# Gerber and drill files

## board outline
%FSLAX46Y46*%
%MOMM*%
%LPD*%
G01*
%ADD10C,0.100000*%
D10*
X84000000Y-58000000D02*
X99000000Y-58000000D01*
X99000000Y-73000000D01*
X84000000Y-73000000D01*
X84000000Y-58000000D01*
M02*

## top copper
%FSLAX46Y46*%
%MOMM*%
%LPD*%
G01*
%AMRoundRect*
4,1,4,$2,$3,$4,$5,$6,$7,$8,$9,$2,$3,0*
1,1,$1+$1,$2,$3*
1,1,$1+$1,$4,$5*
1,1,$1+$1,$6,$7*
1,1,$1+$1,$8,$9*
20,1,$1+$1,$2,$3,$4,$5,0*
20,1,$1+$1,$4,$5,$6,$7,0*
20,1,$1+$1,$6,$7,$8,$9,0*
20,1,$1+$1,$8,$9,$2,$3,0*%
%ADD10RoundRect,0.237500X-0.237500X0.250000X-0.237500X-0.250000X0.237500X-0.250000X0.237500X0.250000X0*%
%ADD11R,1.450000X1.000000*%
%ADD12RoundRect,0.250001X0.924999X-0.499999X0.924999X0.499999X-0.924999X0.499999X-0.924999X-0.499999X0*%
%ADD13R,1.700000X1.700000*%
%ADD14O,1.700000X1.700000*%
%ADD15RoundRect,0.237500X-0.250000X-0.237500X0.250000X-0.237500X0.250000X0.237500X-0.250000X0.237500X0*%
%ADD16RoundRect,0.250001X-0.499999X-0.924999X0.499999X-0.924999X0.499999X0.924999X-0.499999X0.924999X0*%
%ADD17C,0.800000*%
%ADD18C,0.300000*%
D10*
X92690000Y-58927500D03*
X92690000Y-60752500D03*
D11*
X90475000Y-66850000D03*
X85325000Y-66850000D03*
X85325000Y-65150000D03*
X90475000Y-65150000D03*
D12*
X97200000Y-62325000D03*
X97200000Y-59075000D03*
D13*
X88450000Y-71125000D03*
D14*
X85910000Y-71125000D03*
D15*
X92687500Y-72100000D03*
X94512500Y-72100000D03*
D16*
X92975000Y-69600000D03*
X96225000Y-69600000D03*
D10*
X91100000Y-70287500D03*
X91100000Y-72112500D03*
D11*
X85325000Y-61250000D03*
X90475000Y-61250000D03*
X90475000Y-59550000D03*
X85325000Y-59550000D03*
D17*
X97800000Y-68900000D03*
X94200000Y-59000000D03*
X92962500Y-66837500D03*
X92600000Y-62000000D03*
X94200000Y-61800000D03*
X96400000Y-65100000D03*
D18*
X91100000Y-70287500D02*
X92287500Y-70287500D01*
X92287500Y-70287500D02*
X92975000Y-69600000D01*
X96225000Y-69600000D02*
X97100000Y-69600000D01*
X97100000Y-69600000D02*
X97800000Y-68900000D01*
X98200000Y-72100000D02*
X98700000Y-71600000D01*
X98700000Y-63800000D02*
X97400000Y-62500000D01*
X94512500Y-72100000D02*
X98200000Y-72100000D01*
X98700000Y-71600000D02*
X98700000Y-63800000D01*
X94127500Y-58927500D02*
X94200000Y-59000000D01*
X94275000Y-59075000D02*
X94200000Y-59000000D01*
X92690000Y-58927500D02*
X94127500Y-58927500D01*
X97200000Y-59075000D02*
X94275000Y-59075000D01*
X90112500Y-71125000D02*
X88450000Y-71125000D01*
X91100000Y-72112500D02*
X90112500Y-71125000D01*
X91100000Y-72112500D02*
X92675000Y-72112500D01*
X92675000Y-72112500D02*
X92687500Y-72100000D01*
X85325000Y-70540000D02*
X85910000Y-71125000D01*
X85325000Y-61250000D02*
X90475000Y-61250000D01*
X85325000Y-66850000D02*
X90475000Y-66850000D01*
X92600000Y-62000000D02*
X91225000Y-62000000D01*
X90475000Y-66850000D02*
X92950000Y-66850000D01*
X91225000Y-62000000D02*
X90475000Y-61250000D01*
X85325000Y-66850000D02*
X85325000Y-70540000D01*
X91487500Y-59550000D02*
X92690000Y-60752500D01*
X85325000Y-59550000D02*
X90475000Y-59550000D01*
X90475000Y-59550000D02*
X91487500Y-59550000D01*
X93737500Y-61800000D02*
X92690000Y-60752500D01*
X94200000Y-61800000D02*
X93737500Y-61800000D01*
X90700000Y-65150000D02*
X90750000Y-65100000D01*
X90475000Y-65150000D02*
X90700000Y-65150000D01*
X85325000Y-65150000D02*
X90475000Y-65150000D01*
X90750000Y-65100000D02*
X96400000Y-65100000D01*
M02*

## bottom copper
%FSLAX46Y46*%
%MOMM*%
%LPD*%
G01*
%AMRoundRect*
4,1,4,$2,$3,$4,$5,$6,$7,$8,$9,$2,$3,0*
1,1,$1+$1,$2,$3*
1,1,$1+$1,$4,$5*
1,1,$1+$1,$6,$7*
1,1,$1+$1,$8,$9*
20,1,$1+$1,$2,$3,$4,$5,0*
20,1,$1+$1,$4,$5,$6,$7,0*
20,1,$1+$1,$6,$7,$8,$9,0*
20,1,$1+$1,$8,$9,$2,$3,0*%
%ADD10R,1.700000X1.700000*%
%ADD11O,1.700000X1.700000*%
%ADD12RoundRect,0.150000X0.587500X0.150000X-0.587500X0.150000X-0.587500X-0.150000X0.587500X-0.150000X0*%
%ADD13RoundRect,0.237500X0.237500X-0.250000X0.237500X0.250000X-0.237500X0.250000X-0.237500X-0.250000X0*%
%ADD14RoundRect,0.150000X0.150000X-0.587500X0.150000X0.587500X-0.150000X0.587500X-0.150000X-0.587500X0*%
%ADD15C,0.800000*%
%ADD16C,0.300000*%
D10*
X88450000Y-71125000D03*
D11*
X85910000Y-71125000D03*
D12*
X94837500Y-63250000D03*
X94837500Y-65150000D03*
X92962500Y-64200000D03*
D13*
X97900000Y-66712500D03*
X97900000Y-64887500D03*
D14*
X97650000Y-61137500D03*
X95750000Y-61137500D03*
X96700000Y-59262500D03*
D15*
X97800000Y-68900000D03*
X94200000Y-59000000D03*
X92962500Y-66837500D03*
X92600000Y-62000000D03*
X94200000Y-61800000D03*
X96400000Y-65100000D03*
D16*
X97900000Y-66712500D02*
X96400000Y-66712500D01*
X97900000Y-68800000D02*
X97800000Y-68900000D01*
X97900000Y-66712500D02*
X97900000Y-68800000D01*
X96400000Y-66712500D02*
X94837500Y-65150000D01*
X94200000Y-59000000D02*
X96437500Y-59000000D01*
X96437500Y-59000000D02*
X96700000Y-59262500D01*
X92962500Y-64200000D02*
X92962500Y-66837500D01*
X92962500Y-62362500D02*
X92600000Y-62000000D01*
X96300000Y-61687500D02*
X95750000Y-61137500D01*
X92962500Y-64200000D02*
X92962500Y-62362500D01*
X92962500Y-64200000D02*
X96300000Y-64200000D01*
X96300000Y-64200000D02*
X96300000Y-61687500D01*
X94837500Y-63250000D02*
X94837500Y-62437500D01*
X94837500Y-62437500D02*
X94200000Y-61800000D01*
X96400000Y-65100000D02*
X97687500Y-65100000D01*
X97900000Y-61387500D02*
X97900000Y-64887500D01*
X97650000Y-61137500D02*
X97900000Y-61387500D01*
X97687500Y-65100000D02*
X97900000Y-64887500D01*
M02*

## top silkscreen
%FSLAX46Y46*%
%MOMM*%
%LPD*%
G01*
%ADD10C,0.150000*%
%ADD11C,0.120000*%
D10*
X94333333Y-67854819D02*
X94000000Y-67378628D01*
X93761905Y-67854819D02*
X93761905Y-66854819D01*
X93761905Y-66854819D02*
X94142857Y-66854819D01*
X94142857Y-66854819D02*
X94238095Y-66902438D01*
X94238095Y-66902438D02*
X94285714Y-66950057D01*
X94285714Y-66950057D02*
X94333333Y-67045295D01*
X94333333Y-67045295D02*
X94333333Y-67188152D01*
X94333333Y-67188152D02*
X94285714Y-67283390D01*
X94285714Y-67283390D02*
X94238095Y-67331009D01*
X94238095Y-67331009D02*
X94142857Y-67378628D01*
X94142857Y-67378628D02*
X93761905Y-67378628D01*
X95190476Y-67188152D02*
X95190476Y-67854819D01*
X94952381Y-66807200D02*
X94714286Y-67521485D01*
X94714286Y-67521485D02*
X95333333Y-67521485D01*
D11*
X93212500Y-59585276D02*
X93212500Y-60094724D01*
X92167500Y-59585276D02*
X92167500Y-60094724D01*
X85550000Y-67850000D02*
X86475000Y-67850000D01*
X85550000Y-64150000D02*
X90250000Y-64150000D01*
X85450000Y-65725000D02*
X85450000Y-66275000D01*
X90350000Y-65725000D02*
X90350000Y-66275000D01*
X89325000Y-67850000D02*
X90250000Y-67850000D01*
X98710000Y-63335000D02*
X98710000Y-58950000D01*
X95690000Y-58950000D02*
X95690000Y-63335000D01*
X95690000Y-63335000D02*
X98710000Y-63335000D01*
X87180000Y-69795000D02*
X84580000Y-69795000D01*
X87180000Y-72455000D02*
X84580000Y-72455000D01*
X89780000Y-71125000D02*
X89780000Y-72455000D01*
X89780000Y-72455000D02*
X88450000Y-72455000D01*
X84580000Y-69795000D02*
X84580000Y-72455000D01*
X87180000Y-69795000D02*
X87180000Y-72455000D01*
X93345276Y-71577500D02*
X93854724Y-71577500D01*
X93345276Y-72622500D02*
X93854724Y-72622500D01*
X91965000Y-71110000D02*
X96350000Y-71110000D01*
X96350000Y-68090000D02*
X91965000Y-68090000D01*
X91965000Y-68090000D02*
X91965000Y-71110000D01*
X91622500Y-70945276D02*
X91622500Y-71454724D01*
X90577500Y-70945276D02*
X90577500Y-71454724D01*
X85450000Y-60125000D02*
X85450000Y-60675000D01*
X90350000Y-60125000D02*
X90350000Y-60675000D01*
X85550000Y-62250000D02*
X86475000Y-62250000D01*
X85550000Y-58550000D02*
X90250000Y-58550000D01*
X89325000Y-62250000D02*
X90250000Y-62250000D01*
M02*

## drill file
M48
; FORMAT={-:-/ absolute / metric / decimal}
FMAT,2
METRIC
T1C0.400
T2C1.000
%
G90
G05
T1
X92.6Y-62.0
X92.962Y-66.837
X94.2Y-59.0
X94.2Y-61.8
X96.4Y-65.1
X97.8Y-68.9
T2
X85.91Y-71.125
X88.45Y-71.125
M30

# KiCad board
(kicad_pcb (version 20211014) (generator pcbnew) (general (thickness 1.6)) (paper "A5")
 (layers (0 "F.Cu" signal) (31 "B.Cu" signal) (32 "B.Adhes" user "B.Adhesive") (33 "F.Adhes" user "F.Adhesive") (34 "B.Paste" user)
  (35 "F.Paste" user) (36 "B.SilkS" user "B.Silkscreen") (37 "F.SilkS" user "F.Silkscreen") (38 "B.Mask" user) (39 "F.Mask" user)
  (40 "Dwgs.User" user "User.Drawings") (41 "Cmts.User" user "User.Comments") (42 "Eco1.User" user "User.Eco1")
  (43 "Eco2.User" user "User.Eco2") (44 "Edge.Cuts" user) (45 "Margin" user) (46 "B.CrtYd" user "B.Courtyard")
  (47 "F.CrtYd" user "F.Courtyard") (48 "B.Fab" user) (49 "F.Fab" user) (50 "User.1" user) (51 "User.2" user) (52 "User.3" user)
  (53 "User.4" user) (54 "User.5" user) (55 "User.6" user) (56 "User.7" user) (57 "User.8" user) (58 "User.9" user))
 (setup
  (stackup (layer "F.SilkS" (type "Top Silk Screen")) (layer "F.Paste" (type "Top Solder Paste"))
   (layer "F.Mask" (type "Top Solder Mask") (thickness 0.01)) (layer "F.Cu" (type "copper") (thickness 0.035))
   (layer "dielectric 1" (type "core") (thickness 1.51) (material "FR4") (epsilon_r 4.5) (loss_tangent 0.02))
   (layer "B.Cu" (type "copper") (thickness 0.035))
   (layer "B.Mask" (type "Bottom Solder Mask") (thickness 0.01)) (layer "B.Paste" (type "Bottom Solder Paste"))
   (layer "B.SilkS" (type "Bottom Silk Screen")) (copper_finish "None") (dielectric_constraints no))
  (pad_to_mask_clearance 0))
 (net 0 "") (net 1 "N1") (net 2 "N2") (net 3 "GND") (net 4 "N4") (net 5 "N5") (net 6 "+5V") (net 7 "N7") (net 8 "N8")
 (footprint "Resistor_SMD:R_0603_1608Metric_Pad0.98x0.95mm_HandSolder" (layer "F.Cu") (at 92.69 59.84 -90)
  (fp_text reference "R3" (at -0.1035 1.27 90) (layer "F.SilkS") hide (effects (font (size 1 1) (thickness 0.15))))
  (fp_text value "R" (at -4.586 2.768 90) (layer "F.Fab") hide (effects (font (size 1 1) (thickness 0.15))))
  (fp_line (start -0.254724 -0.5225) (end 0.254724 -0.5225) (layer "F.SilkS") (width 0.12))
  (fp_line (start -0.254724 0.5225) (end 0.254724 0.5225) (layer "F.SilkS") (width 0.12))
  (pad "1" smd roundrect (at -0.9125 0 270) (size 0.975 0.95) (layers "F.Cu" "F.Paste" "F.Mask") (roundrect_rratio 0.25) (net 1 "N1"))
  (pad "2" smd roundrect (at 0.9125 0 270) (size 0.975 0.95) (layers "F.Cu" "F.Paste" "F.Mask") (roundrect_rratio 0.25) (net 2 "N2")))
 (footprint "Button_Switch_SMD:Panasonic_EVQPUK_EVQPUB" (layer "F.Cu") (at 87.9 66 180)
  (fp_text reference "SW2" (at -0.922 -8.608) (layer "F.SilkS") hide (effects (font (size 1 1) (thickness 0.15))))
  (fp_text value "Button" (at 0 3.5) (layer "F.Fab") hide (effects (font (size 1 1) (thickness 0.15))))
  (fp_line (start 2.35 -1.85) (end 1.425 -1.85) (layer "F.SilkS") (width 0.12))
  (fp_line (start 2.35 1.85) (end -2.35 1.85) (layer "F.SilkS") (width 0.12))
  (fp_line (start 2.45 0.275) (end 2.45 -0.275) (layer "F.SilkS") (width 0.12))
  (fp_line (start -2.45 0.275) (end -2.45 -0.275) (layer "F.SilkS") (width 0.12))
  (fp_line (start -1.425 -1.85) (end -2.35 -1.85) (layer "F.SilkS") (width 0.12))
  (pad "1" smd rect (at -2.575 -0.85) (size 1.45 1) (layers "F.Cu" "F.Paste" "F.Mask") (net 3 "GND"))
  (pad "1" smd rect (at 2.575 -0.85) (size 1.45 1) (layers "F.Cu" "F.Paste" "F.Mask") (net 3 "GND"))
  (pad "2" smd rect (at 2.575 0.85) (size 1.45 1) (layers "F.Cu" "F.Paste" "F.Mask") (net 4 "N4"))
  (pad "2" smd rect (at -2.575 0.85) (size 1.45 1) (layers "F.Cu" "F.Paste" "F.Mask") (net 4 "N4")))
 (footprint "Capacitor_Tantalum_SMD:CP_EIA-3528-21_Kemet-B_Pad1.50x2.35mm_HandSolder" (layer "F.Cu") (at 97.2 60.7 90)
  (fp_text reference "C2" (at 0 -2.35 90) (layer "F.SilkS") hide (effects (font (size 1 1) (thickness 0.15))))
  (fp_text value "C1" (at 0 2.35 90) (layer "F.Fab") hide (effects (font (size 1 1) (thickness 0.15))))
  (fp_line (start -2.635 1.51) (end 1.75 1.51) (layer "F.SilkS") (width 0.12))
  (fp_line (start 1.75 -1.51) (end -2.635 -1.51) (layer "F.SilkS") (width 0.12))
  (fp_line (start -2.635 -1.51) (end -2.635 1.51) (layer "F.SilkS") (width 0.12))
  (pad "1" smd roundrect (at -1.625 0 90) (size 1.5 2.35) (layers "F.Cu" "F.Paste" "F.Mask") (roundrect_rratio 0.166667) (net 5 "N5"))
  (pad "2" smd roundrect (at 1.625 0 90) (size 1.5 2.35) (layers "F.Cu" "F.Paste" "F.Mask") (roundrect_rratio 0.166667) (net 1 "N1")))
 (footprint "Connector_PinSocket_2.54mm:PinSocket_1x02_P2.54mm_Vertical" (layer "F.Cu") (at 88.45 71.125 -90)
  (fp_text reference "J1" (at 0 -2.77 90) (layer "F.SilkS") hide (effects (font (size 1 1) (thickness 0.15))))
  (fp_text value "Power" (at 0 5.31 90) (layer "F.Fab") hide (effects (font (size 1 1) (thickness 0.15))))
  (fp_line (start -1.33 1.27) (end -1.33 3.87) (layer "F.SilkS") (width 0.12))
  (fp_line (start 1.33 1.27) (end 1.33 3.87) (layer "F.SilkS") (width 0.12))
  (fp_line (start 0 -1.33) (end 1.33 -1.33) (layer "F.SilkS") (width 0.12))
  (fp_line (start 1.33 -1.33) (end 1.33 0) (layer "F.SilkS") (width 0.12))
  (fp_line (start -1.33 3.87) (end 1.33 3.87) (layer "F.SilkS") (width 0.12))
  (fp_line (start -1.33 1.27) (end 1.33 1.27) (layer "F.SilkS") (width 0.12))
  (pad "1" thru_hole rect (at 0 0 270) (size 1.7 1.7) (drill 1) (layers *.Cu *.Mask) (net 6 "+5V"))
  (pad "2" thru_hole oval (at 0 2.54 270) (size 1.7 1.7) (drill 1) (layers *.Cu *.Mask) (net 3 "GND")))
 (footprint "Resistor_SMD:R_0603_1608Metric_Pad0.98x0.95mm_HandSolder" (layer "F.Cu") (at 93.6 72.1)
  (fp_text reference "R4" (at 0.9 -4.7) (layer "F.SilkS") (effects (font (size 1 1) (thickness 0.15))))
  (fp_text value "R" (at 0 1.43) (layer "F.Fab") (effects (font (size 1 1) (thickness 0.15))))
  (fp_line (start -0.254724 -0.5225) (end 0.254724 -0.5225) (layer "F.SilkS") (width 0.12))
  (fp_line (start -0.254724 0.5225) (end 0.254724 0.5225) (layer "F.SilkS") (width 0.12))
  (pad "1" smd roundrect (at -0.9125 0) (size 0.975 0.95) (layers "F.Cu" "F.Paste" "F.Mask") (roundrect_rratio 0.25) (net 6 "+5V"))
  (pad "2" smd roundrect (at 0.9125 0) (size 0.975 0.95) (layers "F.Cu" "F.Paste" "F.Mask") (roundrect_rratio 0.25) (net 5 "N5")))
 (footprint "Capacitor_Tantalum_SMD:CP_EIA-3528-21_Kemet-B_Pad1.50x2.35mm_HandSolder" (layer "F.Cu") (at 94.6 69.6)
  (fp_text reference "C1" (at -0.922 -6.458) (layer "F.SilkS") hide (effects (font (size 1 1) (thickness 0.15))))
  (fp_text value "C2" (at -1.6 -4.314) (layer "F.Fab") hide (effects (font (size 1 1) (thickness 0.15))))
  (fp_line (start -2.635 1.51) (end 1.75 1.51) (layer "F.SilkS") (width 0.12))
  (fp_line (start 1.75 -1.51) (end -2.635 -1.51) (layer "F.SilkS") (width 0.12))
  (fp_line (start -2.635 -1.51) (end -2.635 1.51) (layer "F.SilkS") (width 0.12))
  (pad "1" smd roundrect (at -1.625 0) (size 1.5 2.35) (layers "F.Cu" "F.Paste" "F.Mask") (roundrect_rratio 0.166667) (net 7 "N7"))
  (pad "2" smd roundrect (at 1.625 0) (size 1.5 2.35) (layers "F.Cu" "F.Paste" "F.Mask") (roundrect_rratio 0.166667) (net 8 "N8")))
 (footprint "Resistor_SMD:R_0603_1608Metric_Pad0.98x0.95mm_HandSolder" (layer "F.Cu") (at 91.1 71.2 -90)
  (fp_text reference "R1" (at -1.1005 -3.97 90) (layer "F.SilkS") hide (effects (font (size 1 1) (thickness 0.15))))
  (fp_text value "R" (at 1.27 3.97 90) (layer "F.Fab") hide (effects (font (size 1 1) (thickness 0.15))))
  (fp_line (start -0.254724 -0.5225) (end 0.254724 -0.5225) (layer "F.SilkS") (width 0.12))
  (fp_line (start -0.254724 0.5225) (end 0.254724 0.5225) (layer "F.SilkS") (width 0.12))
  (pad "1" smd roundrect (at -0.9125 0 270) (size 0.975 0.95) (layers "F.Cu" "F.Paste" "F.Mask") (roundrect_rratio 0.25) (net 7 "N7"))
  (pad "2" smd roundrect (at 0.9125 0 270) (size 0.975 0.95) (layers "F.Cu" "F.Paste" "F.Mask") (roundrect_rratio 0.25) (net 6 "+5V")))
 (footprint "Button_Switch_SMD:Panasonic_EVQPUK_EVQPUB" (layer "F.Cu") (at 87.9 60.4 180)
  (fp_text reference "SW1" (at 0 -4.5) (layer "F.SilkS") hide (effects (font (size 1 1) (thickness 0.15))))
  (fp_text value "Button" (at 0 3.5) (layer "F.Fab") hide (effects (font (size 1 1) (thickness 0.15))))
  (fp_line (start 2.45 0.275) (end 2.45 -0.275) (layer "F.SilkS") (width 0.12))
  (fp_line (start -2.45 0.275) (end -2.45 -0.275) (layer "F.SilkS") (width 0.12))
  (fp_line (start 2.35 -1.85) (end 1.425 -1.85) (layer "F.SilkS") (width 0.12))
  (fp_line (start 2.35 1.85) (end -2.35 1.85) (layer "F.SilkS") (width 0.12))
  (fp_line (start -1.425 -1.85) (end -2.35 -1.85) (layer "F.SilkS") (width 0.12))
  (pad "1" smd rect (at 2.575 -0.85) (size 1.45 1) (layers "F.Cu" "F.Paste" "F.Mask") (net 3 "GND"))
  (pad "1" smd rect (at -2.575 -0.85) (size 1.45 1) (layers "F.Cu" "F.Paste" "F.Mask") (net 3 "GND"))
  (pad "2" smd rect (at -2.575 0.85) (size 1.45 1) (layers "F.Cu" "F.Paste" "F.Mask") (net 2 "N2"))
  (pad "2" smd rect (at 2.575 0.85) (size 1.45 1) (layers "F.Cu" "F.Paste" "F.Mask") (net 2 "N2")))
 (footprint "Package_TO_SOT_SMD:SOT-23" (layer "B.Cu") (at 93.9 64.2 180)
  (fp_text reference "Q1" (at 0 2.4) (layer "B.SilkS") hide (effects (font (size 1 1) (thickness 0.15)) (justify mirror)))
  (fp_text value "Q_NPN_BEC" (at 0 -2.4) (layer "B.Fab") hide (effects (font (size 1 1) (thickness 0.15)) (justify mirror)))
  (pad "1" smd roundrect (at -0.9375 0.95 180) (size 1.475 0.6) (layers "B.Cu" "B.Paste" "B.Mask") (roundrect_rratio 0.25) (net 2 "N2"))
  (pad "2" smd roundrect (at -0.9375 -0.95 180) (size 1.475 0.6) (layers "B.Cu" "B.Paste" "B.Mask") (roundrect_rratio 0.25) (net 8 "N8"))
  (pad "3" smd roundrect (at 0.9375 0 180) (size 1.475 0.6) (layers "B.Cu" "B.Paste" "B.Mask") (roundrect_rratio 0.25) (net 3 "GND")))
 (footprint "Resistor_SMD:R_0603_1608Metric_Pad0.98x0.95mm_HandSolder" (layer "B.Cu") (at 97.9 65.8 90)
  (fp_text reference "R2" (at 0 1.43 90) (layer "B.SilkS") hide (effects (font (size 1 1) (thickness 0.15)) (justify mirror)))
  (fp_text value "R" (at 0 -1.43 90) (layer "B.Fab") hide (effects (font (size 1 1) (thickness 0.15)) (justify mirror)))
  (pad "1" smd roundrect (at -0.9125 0 90) (size 0.975 0.95) (layers "B.Cu" "B.Paste" "B.Mask") (roundrect_rratio 0.25) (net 8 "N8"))
  (pad "2" smd roundrect (at 0.9125 0 90) (size 0.975 0.95) (layers "B.Cu" "B.Paste" "B.Mask") (roundrect_rratio 0.25) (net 4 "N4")))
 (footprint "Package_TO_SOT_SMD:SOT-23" (layer "B.Cu") (at 96.7 60.2 90)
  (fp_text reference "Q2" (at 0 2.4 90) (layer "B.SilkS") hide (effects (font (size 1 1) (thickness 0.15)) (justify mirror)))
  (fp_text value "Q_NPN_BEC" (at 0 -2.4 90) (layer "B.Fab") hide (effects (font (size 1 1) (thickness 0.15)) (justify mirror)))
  (pad "1" smd roundrect (at -0.9375 0.95 90) (size 1.475 0.6) (layers "B.Cu" "B.Paste" "B.Mask") (roundrect_rratio 0.25) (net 4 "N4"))
  (pad "2" smd roundrect (at -0.9375 -0.95 90) (size 1.475 0.6) (layers "B.Cu" "B.Paste" "B.Mask") (roundrect_rratio 0.25) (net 3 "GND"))
  (pad "3" smd roundrect (at 0.9375 0 90) (size 1.475 0.6) (layers "B.Cu" "B.Paste" "B.Mask") (roundrect_rratio 0.25) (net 1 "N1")))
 (gr_rect (start 84 58) (end 99 73) (layer "Edge.Cuts") (width 0.1) (fill none))
 (segment (start 91.1 70.2875) (end 92.2875 70.2875) (width 0.3) (layer "F.Cu") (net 7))
 (segment (start 92.2875 70.2875) (end 92.975 69.6) (width 0.3) (layer "F.Cu") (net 7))
 (segment (start 96.225 69.6) (end 97.1 69.6) (width 0.3) (layer "F.Cu") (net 8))
 (segment (start 97.1 69.6) (end 97.8 68.9) (width 0.3) (layer "F.Cu") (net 8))
 (via (at 97.8 68.9) (size 0.8) (drill 0.4) (layers "F.Cu" "B.Cu") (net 8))
 (segment (start 97.9 66.7125) (end 96.4 66.7125) (width 0.3) (layer "B.Cu") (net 8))
 (segment (start 97.9 68.8) (end 97.8 68.9) (width 0.3) (layer "B.Cu") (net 8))
 (segment (start 97.9 66.7125) (end 97.9 68.8) (width 0.3) (layer "B.Cu") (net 8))
 (segment (start 96.4 66.7125) (end 94.8375 65.15) (width 0.3) (layer "B.Cu") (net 8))
 (segment (start 98.2 72.1) (end 98.7 71.6) (width 0.3) (layer "F.Cu") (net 5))
 (segment (start 98.7 63.8) (end 97.4 62.5) (width 0.3) (layer "F.Cu") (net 5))
 (segment (start 94.5125 72.1) (end 98.2 72.1) (width 0.3) (layer "F.Cu") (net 5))
 (segment (start 98.7 71.6) (end 98.7 63.8) (width 0.3) (layer "F.Cu") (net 5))
 (segment (start 94.1275 58.9275) (end 94.2 59) (width 0.3) (layer "F.Cu") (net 1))
 (segment (start 94.275 59.075) (end 94.2 59) (width 0.3) (layer "F.Cu") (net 1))
 (segment (start 92.69 58.9275) (end 94.1275 58.9275) (width 0.3) (layer "F.Cu") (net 1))
 (segment (start 97.2 59.075) (end 94.275 59.075) (width 0.3) (layer "F.Cu") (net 1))
 (via (at 94.2 59) (size 0.8) (drill 0.4) (layers "F.Cu" "B.Cu") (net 1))
 (segment (start 94.2 59) (end 96.4375 59) (width 0.3) (layer "B.Cu") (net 1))
 (segment (start 96.4375 59) (end 96.7 59.2625) (width 0.3) (layer "B.Cu") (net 1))
 (segment (start 90.1125 71.125) (end 88.45 71.125) (width 0.3) (layer "F.Cu") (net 6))
 (segment (start 91.1 72.1125) (end 90.1125 71.125) (width 0.3) (layer "F.Cu") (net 6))
 (segment (start 91.1 72.1125) (end 92.675 72.1125) (width 0.3) (layer "F.Cu") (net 6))
 (segment (start 92.675 72.1125) (end 92.6875 72.1) (width 0.3) (layer "F.Cu") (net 6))
 (segment (start 85.325 70.54) (end 85.91 71.125) (width 0.3) (layer "F.Cu") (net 3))
 (segment (start 85.325 61.25) (end 90.475 61.25) (width 0.3) (layer "F.Cu") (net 3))
 (segment (start 85.325 66.85) (end 90.475 66.85) (width 0.3) (layer "F.Cu") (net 3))
 (segment (start 92.6 62) (end 91.225 62) (width 0.3) (layer "F.Cu") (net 3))
 (segment (start 90.475 66.85) (end 92.95 66.85) (width 0.3) (layer "F.Cu") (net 3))
 (segment (start 91.225 62) (end 90.475 61.25) (width 0.3) (layer "F.Cu") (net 3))
 (segment (start 85.325 66.85) (end 85.325 70.54) (width 0.3) (layer "F.Cu") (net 3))
 (via (at 92.9625 66.8375) (size 0.8) (drill 0.4) (layers "F.Cu" "B.Cu") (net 3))
 (via (at 92.6 62) (size 0.8) (drill 0.4) (layers "F.Cu" "B.Cu") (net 3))
 (segment (start 92.9625 64.2) (end 92.9625 66.8375) (width 0.3) (layer "B.Cu") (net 3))
 (segment (start 92.9625 62.3625) (end 92.6 62) (width 0.3) (layer "B.Cu") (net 3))
 (segment (start 96.3 61.6875) (end 95.75 61.1375) (width 0.3) (layer "B.Cu") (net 3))
 (segment (start 92.9625 64.2) (end 92.9625 62.3625) (width 0.3) (layer "B.Cu") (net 3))
 (segment (start 92.9625 64.2) (end 96.3 64.2) (width 0.3) (layer "B.Cu") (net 3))
 (segment (start 96.3 64.2) (end 96.3 61.6875) (width 0.3) (layer "B.Cu") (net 3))
 (segment (start 91.4875 59.55) (end 92.69 60.7525) (width 0.3) (layer "F.Cu") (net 2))
 (segment (start 85.325 59.55) (end 90.475 59.55) (width 0.3) (layer "F.Cu") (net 2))
 (segment (start 90.475 59.55) (end 91.4875 59.55) (width 0.3) (layer "F.Cu") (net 2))
 (segment (start 93.7375 61.8) (end 92.69 60.7525) (width 0.3) (layer "F.Cu") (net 2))
 (segment (start 94.2 61.8) (end 93.7375 61.8) (width 0.3) (layer "F.Cu") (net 2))
 (via (at 94.2 61.8) (size 0.8) (drill 0.4) (layers "F.Cu" "B.Cu") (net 2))
 (segment (start 94.8375 63.25) (end 94.8375 62.4375) (width 0.3) (layer "B.Cu") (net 2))
 (segment (start 94.8375 62.4375) (end 94.2 61.8) (width 0.3) (layer "B.Cu") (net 2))
 (segment (start 90.7 65.15) (end 90.75 65.1) (width 0.3) (layer "F.Cu") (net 4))
 (segment (start 90.475 65.15) (end 90.7 65.15) (width 0.3) (layer "F.Cu") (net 4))
 (segment (start 85.325 65.15) (end 90.475 65.15) (width 0.3) (layer "F.Cu") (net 4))
 (segment (start 90.75 65.1) (end 96.4 65.1) (width 0.3) (layer "F.Cu") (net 4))
 (via (at 96.4 65.1) (size 0.8) (drill 0.4) (layers "F.Cu" "B.Cu") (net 4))
 (segment (start 96.4 65.1) (end 97.6875 65.1) (width 0.3) (layer "B.Cu") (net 4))
 (segment (start 97.9 61.3875) (end 97.9 64.8875) (width 0.3) (layer "B.Cu") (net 4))
 (segment (start 97.65 61.1375) (end 97.9 61.3875) (width 0.3) (layer "B.Cu") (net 4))
 (segment (start 97.6875 65.1) (end 97.9 64.8875) (width 0.3) (layer "B.Cu") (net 4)))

